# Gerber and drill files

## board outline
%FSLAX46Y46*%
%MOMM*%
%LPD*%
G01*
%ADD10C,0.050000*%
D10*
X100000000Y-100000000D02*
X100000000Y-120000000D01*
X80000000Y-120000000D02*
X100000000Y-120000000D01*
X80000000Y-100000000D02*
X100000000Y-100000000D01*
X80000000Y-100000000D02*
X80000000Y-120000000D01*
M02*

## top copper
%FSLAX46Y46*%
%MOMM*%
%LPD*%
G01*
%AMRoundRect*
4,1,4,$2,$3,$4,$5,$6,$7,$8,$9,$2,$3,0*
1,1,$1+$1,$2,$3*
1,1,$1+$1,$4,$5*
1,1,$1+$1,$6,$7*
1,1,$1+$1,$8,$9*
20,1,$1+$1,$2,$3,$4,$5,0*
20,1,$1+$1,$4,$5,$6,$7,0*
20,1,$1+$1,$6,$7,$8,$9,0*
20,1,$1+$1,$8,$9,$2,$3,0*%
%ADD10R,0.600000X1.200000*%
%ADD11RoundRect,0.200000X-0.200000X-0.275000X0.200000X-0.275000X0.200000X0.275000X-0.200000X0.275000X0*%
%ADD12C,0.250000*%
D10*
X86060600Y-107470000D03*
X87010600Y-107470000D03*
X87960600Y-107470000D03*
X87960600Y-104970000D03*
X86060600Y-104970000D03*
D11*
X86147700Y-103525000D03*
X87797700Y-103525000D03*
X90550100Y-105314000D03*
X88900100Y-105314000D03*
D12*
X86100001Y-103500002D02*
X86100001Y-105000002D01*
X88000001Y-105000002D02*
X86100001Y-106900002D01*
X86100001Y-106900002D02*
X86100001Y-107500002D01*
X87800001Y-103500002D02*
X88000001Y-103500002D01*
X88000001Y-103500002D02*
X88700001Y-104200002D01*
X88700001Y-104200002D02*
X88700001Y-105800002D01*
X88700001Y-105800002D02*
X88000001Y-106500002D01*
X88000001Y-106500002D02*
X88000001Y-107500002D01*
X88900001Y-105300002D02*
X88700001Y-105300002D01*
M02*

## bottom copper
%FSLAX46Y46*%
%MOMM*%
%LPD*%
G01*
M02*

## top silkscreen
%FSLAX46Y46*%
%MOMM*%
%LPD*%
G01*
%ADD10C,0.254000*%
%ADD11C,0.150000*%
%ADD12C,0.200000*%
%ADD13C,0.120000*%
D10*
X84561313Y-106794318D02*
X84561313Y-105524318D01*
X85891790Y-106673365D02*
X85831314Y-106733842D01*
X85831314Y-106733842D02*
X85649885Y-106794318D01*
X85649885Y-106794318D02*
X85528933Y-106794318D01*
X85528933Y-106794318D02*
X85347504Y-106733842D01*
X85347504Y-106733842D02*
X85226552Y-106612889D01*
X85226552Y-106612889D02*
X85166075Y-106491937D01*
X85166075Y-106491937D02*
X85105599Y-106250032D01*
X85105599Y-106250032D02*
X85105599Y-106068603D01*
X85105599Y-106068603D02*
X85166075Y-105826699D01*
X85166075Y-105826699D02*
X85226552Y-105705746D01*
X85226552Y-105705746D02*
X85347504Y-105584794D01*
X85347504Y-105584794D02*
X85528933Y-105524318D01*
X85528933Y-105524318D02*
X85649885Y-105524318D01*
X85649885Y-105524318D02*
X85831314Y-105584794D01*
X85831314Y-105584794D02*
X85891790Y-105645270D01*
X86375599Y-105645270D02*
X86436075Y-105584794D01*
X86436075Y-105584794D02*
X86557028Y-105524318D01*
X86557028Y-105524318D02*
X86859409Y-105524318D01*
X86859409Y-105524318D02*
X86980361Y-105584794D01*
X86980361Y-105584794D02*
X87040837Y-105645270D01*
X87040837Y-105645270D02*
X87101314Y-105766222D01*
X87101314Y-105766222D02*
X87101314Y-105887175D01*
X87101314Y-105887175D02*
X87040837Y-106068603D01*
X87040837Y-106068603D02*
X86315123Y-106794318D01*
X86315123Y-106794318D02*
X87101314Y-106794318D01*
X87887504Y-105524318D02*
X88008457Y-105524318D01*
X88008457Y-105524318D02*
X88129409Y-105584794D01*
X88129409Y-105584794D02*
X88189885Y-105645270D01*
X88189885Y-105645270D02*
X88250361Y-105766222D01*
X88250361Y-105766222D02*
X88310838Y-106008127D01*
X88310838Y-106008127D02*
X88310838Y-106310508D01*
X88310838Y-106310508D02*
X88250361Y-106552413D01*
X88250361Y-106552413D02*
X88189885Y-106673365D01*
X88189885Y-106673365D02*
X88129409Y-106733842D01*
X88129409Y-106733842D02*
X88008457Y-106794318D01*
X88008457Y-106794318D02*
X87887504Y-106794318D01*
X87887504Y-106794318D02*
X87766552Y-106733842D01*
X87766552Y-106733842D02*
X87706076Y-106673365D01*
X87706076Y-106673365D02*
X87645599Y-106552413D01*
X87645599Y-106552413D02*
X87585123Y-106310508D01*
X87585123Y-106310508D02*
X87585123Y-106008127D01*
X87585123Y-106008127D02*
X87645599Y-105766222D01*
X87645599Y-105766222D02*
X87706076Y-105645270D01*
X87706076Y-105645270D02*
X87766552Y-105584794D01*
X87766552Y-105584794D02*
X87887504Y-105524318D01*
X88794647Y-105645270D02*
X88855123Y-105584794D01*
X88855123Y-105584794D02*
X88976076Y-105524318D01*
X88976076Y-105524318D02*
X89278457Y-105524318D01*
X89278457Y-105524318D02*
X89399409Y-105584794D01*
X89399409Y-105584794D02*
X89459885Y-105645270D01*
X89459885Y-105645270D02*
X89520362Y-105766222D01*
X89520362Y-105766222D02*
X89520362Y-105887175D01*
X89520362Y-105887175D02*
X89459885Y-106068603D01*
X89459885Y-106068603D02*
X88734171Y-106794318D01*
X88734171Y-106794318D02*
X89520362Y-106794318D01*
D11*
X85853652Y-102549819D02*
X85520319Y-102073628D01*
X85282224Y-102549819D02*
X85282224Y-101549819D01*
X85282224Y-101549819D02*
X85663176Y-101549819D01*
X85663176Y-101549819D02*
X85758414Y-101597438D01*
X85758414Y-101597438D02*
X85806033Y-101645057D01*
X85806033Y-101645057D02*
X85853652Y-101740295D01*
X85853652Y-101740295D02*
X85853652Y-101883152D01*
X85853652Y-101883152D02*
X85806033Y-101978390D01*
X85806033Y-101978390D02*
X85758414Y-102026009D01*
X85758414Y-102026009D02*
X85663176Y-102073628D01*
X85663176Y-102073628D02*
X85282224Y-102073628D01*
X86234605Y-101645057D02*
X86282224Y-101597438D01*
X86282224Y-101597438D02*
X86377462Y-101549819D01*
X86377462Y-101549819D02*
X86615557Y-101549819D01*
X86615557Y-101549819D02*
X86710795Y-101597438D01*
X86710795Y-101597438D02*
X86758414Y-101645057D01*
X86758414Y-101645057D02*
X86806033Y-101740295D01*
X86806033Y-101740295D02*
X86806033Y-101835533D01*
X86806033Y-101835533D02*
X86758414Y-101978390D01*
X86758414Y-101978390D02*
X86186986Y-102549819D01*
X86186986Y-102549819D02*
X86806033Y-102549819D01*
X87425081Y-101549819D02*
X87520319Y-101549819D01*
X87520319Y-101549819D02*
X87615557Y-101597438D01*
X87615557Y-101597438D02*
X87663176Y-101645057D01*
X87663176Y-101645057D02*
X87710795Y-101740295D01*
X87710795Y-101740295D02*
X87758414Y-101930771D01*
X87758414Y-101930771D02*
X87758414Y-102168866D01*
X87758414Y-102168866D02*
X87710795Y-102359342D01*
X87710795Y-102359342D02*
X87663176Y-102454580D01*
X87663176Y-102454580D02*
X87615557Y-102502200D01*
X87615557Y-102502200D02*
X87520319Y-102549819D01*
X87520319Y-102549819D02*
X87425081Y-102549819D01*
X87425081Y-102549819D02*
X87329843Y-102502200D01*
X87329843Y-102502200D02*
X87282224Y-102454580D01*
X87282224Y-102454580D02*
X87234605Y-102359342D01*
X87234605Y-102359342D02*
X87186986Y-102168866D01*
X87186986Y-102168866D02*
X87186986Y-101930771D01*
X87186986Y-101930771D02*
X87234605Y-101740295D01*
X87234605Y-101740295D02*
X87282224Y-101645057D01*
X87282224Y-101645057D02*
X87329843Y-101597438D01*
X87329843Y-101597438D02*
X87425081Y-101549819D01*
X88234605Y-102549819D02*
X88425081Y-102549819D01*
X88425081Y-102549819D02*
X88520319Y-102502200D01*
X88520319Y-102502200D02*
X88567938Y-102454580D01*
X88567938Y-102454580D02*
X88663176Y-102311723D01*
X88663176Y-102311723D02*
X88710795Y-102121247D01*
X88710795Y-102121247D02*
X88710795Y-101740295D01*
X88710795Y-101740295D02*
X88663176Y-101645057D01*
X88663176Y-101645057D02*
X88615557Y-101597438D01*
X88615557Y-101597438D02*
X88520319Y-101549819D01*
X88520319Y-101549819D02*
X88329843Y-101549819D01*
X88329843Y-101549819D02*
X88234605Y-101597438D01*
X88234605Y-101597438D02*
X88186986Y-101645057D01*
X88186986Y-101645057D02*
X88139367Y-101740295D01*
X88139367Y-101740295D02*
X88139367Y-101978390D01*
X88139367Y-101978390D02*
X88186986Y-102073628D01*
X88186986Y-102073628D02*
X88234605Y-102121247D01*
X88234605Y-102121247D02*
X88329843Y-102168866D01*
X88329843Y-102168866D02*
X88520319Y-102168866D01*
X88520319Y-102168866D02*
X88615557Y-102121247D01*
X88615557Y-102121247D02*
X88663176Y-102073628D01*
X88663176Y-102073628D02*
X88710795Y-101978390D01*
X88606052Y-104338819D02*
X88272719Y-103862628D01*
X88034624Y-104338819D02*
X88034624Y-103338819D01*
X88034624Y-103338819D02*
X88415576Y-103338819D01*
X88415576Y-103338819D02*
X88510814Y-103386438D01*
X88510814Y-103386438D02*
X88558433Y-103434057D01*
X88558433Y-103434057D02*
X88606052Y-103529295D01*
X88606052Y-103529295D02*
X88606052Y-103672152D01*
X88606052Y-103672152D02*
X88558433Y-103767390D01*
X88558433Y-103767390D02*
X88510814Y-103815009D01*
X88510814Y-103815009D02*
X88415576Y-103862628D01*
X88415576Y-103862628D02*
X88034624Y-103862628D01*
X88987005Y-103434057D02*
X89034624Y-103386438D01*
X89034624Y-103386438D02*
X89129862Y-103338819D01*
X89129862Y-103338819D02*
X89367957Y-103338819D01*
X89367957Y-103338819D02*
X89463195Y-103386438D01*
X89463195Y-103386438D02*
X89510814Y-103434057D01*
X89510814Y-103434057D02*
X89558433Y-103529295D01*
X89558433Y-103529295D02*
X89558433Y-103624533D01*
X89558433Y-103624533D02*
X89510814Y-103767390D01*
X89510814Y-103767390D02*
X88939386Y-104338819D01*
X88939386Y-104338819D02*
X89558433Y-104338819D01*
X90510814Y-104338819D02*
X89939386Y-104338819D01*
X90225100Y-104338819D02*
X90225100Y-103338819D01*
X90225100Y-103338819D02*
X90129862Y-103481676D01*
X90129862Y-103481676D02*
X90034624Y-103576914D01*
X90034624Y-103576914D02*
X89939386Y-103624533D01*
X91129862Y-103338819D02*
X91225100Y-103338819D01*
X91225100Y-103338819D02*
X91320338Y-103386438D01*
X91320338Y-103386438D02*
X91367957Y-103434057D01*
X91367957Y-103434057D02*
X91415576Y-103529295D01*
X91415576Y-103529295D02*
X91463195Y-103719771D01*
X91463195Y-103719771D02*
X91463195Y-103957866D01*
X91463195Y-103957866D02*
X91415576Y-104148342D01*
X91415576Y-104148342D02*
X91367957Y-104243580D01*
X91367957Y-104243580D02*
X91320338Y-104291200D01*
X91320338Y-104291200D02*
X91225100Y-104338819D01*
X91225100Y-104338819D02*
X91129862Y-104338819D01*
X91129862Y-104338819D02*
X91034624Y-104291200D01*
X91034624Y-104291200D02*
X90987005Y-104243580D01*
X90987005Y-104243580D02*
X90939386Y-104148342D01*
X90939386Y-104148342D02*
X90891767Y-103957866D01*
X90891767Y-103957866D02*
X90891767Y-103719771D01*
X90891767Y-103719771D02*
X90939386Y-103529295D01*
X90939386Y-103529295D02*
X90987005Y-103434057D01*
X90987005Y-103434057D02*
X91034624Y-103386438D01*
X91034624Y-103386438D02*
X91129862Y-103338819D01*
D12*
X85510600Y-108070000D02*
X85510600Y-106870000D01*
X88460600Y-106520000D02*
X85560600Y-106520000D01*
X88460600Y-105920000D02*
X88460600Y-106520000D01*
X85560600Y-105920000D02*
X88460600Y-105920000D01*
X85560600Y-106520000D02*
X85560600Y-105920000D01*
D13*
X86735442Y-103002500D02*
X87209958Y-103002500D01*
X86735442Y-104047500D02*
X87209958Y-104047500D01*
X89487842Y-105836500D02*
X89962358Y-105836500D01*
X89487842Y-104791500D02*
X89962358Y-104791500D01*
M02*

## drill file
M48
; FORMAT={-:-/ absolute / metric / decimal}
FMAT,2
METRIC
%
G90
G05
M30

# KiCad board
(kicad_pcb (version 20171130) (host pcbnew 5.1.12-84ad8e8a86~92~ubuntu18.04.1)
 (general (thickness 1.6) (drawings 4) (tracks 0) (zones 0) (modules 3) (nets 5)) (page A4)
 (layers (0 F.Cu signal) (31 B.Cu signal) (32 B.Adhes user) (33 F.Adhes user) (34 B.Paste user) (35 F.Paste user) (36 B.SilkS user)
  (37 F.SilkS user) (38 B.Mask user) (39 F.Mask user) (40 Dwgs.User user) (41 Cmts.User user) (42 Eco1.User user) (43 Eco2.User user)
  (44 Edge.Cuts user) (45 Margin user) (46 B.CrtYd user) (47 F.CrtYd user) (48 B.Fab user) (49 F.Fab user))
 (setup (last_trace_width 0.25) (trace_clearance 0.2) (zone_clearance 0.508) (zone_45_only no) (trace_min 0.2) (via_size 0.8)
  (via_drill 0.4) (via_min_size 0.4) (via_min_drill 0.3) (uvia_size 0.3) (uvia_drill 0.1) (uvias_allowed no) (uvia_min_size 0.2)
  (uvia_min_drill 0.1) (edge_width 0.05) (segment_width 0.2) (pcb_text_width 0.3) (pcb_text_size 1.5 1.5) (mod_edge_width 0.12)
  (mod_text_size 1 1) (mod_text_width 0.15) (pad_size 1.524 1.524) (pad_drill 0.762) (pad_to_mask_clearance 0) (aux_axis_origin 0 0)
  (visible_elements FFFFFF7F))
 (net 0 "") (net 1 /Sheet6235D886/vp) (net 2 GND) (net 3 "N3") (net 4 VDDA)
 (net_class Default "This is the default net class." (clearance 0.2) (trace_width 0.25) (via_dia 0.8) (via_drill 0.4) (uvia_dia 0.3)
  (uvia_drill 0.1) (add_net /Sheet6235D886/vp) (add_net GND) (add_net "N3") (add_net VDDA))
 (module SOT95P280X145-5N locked (layer F.Cu) (at 87.010600 106.220000 90.000000)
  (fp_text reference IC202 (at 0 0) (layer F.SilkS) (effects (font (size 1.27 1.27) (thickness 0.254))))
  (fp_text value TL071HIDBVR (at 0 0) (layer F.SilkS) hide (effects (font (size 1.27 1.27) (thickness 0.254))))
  (fp_line (start -1.85 -1.5) (end -0.65 -1.5) (layer F.SilkS) (width 0.2))
  (fp_line (start -0.3 1.45) (end -0.3 -1.45) (layer F.SilkS) (width 0.2))
  (fp_line (start 0.3 1.45) (end -0.3 1.45) (layer F.SilkS) (width 0.2))
  (fp_line (start 0.3 -1.45) (end 0.3 1.45) (layer F.SilkS) (width 0.2))
  (fp_line (start -0.3 -1.45) (end 0.3 -1.45) (layer F.SilkS) (width 0.2))
  (pad 1 smd rect (at -1.25 -0.95 180.000000) (size 0.6 1.2) (layers F.Cu F.Mask F.Paste) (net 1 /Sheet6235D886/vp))
  (pad 2 smd rect (at -1.25 0 180.000000) (size 0.6 1.2) (layers F.Cu F.Mask F.Paste) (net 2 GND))
  (pad 3 smd rect (at -1.25 0.95 180.000000) (size 0.6 1.2) (layers F.Cu F.Mask F.Paste) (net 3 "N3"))
  (pad 4 smd rect (at 1.25 0.95 180.000000) (size 0.6 1.2) (layers F.Cu F.Mask F.Paste) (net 1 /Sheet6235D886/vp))
  (pad 5 smd rect (at 1.25 -0.95 180.000000) (size 0.6 1.2) (layers F.Cu F.Mask F.Paste) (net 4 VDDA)))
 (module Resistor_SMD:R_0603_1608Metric (layer F.Cu) (at 86.972700 103.525000)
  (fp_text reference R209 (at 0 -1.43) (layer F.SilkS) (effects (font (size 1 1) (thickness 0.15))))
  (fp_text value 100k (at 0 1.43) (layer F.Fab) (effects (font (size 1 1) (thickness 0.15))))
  (fp_line (start -0.237258 -0.5225) (end 0.237258 -0.5225) (layer F.SilkS) (width 0.12))
  (fp_line (start -0.237258 0.5225) (end 0.237258 0.5225) (layer F.SilkS) (width 0.12))
  (pad 1 smd roundrect (at -0.825 0) (size 0.8 0.95) (layers F.Cu F.Mask F.Paste) (roundrect_rratio 0.25) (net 4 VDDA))
  (pad 2 smd roundrect (at 0.825 0) (size 0.8 0.95) (layers F.Cu F.Mask F.Paste) (roundrect_rratio 0.25) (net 3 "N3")))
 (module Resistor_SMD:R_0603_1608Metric (layer F.Cu) (at 89.725100 105.314000)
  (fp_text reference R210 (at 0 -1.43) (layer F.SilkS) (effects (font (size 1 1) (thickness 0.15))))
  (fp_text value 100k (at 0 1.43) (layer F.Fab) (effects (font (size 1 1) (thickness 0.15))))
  (fp_line (start -0.237258 0.5225) (end 0.237258 0.5225) (layer F.SilkS) (width 0.12))
  (fp_line (start -0.237258 -0.5225) (end 0.237258 -0.5225) (layer F.SilkS) (width 0.12))
  (pad 2 smd roundrect (at 0.825 0) (size 0.8 0.95) (layers F.Cu F.Mask F.Paste) (roundrect_rratio 0.25) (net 2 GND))
  (pad 1 smd roundrect (at -0.825 0) (size 0.8 0.95) (layers F.Cu F.Mask F.Paste) (roundrect_rratio 0.25) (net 3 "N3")))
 (gr_line (start 100 100) (end 100 120) (layer Edge.Cuts) (width 0.05))
 (gr_line (start 80 120) (end 100 120) (layer Edge.Cuts) (width 0.05))
 (gr_line (start 80 100) (end 100 100) (layer Edge.Cuts) (width 0.05))
 (gr_line (start 80 100) (end 80 120) (layer Edge.Cuts) (width 0.05))
 (segment (start 86.100001 103.500002) (end 86.100001 105.000002) (width 0.250000) (layer F.Cu) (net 4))
 (segment (start 88.000001 105.000002) (end 86.100001 106.900002) (width 0.250000) (layer F.Cu) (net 1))
 (segment (start 86.100001 106.900002) (end 86.100001 107.500002) (width 0.250000) (layer F.Cu) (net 1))
 (segment (start 87.800001 103.500002) (end 88.000001 103.500002) (width 0.250000) (layer F.Cu) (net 3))
 (segment (start 88.000001 103.500002) (end 88.700001 104.200002) (width 0.250000) (layer F.Cu) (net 3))
 (segment (start 88.700001 104.200002) (end 88.700001 105.800002) (width 0.250000) (layer F.Cu) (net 3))
 (segment (start 88.700001 105.800002) (end 88.000001 106.500002) (width 0.250000) (layer F.Cu) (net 3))
 (segment (start 88.000001 106.500002) (end 88.000001 107.500002) (width 0.250000) (layer F.Cu) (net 3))
 (segment (start 88.900001 105.300002) (end 88.700001 105.300002) (width 0.250000) (layer F.Cu) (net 3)))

